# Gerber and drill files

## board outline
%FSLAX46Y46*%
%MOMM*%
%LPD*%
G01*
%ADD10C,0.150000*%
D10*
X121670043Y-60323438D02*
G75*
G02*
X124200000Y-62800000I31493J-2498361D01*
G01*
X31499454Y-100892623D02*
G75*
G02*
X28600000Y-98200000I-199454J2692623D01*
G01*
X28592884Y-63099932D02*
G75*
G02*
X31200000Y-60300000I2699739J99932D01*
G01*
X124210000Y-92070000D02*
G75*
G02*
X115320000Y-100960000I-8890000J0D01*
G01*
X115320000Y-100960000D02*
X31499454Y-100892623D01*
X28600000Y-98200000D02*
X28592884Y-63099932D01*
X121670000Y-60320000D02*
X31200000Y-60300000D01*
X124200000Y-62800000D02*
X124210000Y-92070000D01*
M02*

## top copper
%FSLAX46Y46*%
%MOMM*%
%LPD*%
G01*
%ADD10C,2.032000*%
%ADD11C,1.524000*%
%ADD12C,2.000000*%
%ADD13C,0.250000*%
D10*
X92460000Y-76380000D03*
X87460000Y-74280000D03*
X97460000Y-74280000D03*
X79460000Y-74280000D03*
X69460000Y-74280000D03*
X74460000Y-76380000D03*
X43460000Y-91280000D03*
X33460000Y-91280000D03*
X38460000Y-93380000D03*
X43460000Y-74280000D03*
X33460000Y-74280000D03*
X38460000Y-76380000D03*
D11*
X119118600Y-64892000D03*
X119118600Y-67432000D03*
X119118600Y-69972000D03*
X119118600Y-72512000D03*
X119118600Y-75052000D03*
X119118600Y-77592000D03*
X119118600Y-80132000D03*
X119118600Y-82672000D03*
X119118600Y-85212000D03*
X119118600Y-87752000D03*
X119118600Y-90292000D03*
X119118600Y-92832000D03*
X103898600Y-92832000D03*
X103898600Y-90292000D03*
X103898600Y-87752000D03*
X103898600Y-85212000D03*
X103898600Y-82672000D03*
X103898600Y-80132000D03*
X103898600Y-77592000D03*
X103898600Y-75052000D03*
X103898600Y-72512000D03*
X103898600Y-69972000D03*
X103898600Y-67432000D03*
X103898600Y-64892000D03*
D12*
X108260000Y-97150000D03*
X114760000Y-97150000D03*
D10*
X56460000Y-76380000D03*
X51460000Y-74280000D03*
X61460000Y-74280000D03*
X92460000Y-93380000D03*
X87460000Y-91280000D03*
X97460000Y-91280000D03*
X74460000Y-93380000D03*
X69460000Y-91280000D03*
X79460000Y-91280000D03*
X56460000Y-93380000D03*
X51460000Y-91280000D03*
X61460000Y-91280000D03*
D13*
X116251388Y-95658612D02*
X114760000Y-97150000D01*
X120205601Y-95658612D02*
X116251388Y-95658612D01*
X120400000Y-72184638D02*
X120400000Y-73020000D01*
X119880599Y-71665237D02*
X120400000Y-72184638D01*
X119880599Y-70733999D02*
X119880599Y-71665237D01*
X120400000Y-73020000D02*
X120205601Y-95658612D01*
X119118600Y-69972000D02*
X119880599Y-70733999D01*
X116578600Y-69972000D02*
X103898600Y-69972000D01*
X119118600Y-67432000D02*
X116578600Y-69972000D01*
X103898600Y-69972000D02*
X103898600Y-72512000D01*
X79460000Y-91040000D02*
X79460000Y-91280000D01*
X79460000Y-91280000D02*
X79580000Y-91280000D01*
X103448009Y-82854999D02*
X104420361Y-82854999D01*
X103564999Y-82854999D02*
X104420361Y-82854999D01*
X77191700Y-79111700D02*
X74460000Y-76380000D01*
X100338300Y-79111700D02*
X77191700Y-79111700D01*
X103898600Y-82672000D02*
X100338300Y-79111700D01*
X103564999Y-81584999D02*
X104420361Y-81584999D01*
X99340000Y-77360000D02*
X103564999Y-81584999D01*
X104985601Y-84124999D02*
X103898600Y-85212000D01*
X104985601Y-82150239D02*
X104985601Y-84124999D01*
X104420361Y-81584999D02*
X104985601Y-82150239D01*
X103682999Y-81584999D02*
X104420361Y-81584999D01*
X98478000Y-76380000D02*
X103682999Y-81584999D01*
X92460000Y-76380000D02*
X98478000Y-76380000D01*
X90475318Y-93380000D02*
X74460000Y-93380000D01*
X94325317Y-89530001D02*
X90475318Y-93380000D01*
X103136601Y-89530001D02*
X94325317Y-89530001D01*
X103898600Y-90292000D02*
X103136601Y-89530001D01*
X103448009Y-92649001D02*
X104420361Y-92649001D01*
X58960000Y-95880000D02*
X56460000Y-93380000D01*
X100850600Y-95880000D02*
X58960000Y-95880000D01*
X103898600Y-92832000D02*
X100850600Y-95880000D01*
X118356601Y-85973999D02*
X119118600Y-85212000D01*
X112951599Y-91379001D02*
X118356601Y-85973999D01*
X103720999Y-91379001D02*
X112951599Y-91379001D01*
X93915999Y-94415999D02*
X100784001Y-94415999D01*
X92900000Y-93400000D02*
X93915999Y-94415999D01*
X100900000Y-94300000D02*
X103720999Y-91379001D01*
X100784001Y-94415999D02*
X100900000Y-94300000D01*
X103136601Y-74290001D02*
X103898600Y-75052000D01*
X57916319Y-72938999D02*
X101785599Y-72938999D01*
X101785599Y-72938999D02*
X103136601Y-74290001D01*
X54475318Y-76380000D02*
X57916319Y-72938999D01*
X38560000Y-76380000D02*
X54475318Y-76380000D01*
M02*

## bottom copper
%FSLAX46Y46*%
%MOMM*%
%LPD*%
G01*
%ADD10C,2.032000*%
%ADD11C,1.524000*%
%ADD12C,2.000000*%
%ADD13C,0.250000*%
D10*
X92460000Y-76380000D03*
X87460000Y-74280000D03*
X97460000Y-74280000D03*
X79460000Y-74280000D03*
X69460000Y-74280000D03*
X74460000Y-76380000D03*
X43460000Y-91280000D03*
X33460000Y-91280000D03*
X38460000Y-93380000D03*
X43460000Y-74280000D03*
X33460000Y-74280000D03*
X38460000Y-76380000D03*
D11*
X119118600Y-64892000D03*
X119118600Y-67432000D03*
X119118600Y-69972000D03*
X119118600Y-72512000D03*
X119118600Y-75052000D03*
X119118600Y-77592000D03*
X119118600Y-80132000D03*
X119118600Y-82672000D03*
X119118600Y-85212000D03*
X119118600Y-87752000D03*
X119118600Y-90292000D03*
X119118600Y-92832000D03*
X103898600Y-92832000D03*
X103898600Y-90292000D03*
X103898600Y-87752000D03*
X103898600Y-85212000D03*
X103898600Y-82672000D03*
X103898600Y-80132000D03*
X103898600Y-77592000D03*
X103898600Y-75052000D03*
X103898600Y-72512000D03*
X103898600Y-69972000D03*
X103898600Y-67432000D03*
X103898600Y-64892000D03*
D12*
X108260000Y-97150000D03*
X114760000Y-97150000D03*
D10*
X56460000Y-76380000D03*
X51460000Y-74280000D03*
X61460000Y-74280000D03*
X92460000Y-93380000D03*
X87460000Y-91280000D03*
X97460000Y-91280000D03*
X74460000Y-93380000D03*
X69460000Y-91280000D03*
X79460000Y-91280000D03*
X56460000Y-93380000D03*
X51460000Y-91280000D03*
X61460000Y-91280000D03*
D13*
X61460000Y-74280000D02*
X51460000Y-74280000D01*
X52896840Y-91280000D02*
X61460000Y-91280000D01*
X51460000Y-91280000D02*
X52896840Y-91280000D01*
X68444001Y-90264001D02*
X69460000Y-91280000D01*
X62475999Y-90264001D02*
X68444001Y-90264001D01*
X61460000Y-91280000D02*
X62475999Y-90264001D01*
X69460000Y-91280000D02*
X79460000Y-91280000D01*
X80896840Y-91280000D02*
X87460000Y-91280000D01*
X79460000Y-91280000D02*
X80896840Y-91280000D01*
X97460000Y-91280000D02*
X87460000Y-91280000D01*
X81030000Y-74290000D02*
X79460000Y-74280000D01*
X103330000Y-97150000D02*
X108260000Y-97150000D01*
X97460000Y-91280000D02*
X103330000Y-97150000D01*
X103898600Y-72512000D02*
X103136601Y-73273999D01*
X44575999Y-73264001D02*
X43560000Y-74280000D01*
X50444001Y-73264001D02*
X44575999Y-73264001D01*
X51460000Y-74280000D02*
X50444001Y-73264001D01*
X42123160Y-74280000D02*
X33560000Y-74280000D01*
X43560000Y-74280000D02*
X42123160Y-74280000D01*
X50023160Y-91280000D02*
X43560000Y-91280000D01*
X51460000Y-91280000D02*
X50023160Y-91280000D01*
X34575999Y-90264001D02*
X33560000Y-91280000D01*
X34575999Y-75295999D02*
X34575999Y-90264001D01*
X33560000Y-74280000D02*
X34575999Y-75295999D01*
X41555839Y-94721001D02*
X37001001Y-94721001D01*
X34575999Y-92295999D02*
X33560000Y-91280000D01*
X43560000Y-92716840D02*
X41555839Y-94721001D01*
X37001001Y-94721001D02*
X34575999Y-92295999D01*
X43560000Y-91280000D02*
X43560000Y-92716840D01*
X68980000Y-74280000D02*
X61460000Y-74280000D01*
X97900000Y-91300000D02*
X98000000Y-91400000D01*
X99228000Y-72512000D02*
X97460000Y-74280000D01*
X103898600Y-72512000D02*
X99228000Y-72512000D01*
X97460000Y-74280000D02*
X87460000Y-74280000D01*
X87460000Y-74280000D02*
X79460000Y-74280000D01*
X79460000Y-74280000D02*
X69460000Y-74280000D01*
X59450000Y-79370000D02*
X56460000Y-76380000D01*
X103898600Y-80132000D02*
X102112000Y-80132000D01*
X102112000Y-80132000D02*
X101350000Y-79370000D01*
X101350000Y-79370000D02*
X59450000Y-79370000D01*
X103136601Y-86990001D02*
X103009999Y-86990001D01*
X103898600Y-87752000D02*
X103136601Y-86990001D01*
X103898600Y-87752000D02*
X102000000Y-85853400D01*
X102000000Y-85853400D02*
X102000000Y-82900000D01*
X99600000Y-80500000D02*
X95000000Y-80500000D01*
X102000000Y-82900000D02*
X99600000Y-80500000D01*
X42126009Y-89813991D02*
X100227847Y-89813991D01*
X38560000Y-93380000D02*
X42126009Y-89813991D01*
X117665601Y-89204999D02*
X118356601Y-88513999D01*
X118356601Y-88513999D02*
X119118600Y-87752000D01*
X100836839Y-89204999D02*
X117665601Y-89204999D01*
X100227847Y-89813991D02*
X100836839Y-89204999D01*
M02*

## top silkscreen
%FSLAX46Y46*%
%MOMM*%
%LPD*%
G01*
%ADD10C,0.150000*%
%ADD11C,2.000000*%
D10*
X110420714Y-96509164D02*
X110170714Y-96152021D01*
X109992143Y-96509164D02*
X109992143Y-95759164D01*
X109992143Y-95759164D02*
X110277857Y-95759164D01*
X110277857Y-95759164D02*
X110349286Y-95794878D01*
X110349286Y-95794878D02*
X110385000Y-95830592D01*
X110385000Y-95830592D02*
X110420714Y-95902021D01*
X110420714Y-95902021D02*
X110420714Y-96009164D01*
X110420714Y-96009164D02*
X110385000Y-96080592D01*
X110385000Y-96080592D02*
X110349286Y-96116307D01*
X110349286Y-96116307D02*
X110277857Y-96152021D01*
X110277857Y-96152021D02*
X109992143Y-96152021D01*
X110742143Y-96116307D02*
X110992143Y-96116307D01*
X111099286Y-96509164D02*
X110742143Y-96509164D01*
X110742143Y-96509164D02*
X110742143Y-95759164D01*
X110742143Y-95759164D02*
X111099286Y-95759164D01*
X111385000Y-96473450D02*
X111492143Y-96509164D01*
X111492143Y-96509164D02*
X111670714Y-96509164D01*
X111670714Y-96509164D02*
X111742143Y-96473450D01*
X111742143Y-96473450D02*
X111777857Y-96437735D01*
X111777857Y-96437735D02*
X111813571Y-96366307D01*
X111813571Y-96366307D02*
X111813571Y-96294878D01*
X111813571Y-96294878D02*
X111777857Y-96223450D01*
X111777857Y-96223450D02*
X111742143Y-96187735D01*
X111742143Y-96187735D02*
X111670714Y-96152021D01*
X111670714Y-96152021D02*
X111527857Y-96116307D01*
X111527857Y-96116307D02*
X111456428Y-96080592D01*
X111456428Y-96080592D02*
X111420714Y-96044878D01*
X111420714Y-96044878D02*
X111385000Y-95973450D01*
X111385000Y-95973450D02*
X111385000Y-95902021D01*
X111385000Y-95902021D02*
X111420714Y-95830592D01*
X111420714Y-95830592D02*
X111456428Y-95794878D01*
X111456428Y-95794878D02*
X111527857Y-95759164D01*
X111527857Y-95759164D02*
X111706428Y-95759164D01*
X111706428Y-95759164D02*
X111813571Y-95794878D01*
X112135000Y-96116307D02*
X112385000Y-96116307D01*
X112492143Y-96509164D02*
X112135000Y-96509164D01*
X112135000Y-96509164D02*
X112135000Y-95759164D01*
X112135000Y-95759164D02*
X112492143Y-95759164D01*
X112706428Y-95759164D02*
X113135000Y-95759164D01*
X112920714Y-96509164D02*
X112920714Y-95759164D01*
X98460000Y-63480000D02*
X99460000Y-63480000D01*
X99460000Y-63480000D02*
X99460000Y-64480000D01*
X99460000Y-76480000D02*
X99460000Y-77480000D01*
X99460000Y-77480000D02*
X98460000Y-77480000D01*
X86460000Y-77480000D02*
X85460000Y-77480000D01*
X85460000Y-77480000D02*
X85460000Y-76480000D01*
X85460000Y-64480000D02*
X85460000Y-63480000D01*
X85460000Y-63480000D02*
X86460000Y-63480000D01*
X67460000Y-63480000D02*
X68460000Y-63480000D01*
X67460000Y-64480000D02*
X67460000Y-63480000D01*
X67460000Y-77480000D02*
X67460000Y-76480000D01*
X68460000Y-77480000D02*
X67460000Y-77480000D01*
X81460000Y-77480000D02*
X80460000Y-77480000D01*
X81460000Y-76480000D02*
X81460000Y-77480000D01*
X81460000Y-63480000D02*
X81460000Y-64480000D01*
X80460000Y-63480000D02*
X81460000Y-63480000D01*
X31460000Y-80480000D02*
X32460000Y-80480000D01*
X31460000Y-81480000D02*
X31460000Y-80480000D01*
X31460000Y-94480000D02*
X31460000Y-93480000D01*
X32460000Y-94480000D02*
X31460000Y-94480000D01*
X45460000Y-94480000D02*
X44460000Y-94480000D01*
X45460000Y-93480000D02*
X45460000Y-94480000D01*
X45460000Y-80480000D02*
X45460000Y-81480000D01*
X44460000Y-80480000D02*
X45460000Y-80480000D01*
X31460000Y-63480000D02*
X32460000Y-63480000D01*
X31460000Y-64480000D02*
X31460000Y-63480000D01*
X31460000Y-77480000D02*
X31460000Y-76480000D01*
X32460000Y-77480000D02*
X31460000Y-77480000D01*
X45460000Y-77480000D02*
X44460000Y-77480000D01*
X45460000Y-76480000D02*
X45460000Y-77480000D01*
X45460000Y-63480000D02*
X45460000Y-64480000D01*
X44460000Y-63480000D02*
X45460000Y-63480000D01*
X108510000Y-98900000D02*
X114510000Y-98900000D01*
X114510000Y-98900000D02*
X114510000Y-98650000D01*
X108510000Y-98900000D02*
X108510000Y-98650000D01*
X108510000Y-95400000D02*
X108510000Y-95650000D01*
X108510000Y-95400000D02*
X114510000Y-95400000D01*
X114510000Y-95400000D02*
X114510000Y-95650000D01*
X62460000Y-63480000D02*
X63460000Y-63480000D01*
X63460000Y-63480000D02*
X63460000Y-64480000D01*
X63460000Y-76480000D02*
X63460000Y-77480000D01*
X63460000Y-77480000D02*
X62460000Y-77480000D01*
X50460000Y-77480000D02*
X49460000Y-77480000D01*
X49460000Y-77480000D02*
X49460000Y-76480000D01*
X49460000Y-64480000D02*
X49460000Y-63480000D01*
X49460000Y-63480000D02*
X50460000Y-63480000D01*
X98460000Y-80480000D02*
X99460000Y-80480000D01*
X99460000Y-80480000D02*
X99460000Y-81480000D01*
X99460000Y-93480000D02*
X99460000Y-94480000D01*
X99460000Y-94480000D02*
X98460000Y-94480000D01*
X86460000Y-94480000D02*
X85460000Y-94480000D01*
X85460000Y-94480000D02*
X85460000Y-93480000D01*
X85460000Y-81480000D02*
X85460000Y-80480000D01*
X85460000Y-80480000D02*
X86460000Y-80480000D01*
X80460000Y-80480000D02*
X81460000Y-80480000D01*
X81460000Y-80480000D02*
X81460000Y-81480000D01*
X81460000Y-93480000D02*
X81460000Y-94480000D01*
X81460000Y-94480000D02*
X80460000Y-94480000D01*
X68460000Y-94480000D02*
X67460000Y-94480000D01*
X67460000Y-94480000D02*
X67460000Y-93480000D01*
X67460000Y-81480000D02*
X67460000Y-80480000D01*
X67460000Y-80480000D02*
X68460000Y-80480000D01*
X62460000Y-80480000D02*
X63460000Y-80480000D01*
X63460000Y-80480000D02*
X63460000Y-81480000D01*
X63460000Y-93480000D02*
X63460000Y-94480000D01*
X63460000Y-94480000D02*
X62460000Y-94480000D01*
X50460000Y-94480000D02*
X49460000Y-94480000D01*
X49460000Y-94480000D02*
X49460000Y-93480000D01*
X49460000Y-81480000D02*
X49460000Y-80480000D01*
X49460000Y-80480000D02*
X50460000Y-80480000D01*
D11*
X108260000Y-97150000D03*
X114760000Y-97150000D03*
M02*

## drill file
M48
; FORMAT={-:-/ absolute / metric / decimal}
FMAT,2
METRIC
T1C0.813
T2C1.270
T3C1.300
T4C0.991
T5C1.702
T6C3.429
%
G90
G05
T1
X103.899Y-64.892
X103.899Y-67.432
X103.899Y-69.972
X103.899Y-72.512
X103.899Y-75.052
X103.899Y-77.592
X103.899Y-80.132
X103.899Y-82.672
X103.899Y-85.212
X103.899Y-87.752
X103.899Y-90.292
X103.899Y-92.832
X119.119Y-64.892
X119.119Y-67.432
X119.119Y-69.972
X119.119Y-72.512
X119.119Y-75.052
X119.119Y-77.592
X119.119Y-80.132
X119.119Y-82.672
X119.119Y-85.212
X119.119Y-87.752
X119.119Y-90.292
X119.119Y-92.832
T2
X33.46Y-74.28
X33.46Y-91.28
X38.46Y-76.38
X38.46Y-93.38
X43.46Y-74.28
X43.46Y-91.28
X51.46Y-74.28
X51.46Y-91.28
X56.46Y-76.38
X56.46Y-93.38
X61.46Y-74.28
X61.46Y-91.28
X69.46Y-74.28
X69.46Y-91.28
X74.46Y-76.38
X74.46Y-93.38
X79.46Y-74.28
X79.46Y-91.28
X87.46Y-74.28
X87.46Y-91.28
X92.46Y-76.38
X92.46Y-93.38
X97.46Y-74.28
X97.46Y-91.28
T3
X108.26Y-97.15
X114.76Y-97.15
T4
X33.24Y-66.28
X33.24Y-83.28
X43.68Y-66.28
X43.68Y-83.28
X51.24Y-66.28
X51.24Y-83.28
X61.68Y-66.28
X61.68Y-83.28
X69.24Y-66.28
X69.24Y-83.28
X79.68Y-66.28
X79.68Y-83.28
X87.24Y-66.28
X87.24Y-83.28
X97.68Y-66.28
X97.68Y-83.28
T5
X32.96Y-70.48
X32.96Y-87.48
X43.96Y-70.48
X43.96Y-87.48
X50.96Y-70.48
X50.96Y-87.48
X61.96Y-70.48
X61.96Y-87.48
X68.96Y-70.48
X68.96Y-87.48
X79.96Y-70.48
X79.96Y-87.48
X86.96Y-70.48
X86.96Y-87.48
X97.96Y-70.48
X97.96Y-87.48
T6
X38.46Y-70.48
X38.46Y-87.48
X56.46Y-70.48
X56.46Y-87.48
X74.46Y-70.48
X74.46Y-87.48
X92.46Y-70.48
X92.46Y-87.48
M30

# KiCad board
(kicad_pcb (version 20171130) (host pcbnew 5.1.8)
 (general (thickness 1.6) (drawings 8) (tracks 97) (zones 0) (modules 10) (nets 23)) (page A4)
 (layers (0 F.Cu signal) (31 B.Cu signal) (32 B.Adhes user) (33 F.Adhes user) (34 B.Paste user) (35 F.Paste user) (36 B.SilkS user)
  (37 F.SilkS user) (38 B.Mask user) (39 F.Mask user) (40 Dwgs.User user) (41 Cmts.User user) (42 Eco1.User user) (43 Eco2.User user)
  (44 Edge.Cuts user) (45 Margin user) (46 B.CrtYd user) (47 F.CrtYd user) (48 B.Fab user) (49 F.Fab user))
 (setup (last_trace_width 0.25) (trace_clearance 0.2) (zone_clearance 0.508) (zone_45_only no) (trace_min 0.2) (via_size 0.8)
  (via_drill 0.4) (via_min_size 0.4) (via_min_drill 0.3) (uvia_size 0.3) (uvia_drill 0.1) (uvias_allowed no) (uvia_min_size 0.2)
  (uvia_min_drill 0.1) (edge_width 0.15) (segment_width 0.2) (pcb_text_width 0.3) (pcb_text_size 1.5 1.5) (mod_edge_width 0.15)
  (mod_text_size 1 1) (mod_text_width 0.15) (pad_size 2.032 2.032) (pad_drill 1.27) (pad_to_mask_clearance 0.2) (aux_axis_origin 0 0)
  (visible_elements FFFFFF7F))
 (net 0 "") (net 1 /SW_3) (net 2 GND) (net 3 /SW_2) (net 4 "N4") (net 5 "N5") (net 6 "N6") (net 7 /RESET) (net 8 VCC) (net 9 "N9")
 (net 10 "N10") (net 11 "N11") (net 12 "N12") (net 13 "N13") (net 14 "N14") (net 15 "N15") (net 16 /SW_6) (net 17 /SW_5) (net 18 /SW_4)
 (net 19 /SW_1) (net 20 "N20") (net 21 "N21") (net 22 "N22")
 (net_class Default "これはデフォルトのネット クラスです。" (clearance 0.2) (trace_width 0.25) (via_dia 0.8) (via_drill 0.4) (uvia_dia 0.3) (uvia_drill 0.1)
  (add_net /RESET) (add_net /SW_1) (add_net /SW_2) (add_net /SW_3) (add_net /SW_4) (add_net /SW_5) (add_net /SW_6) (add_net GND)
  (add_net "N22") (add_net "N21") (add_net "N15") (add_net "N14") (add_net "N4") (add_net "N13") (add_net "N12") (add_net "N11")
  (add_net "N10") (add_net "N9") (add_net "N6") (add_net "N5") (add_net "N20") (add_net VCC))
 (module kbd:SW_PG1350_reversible (layer F.Cu) (at 92.46 70.48)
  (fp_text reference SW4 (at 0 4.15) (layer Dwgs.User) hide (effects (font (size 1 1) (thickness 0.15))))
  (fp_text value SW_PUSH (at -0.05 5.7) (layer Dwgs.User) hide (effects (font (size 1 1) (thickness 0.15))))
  (fp_line (start 6 -7) (end 7 -7) (layer F.SilkS) (width 0.15))
  (fp_line (start 7 -7) (end 7 -6) (layer F.SilkS) (width 0.15)) (fp_line (start 7 6) (end 7 7) (layer F.SilkS) (width 0.15))
  (fp_line (start 7 7) (end 6 7) (layer F.SilkS) (width 0.15))
  (fp_line (start -6 7) (end -7 7) (layer F.SilkS) (width 0.15))
  (fp_line (start -7 7) (end -7 6) (layer F.SilkS) (width 0.15))
  (fp_line (start -7 -6) (end -7 -7) (layer F.SilkS) (width 0.15))
  (fp_line (start -7 -7) (end -6 -7) (layer F.SilkS) (width 0.15))
  (pad "" np_thru_hole circle (at -5.5 0) (size 1.7018 1.7018) (drill 1.7018) (layers *.Cu *.Mask))
  (pad "" np_thru_hole circle (at 5.5 0) (size 1.7018 1.7018) (drill 1.7018) (layers *.Cu *.Mask))
  (pad "" np_thru_hole circle (at 5.22 -4.2) (size 0.9906 0.9906) (drill 0.9906) (layers *.Cu *.Mask))
  (pad 1 thru_hole circle (at 0 5.9) (size 2.032 2.032) (drill 1.27) (layers *.Cu *.Mask) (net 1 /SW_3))
  (pad 2 thru_hole circle (at -5 3.8) (size 2.032 2.032) (drill 1.27) (layers *.Cu *.Mask) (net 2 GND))
  (pad "" np_thru_hole circle (at 0 0) (size 3.429 3.429) (drill 3.429) (layers *.Cu *.Mask))
  (pad 2 thru_hole circle (at 5 3.8) (size 2.032 2.032) (drill 1.27) (layers *.Cu *.Mask) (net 2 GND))
  (pad "" np_thru_hole circle (at -5.22 -4.2) (size 0.9906 0.9906) (drill 0.9906) (layers *.Cu *.Mask)))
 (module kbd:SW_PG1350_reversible (layer F.Cu) (at 74.46 70.48)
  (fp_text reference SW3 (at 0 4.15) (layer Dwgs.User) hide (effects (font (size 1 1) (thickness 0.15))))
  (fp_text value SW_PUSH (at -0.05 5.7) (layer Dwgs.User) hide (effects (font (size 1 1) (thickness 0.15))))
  (fp_line (start -7 -7) (end -6 -7) (layer F.SilkS) (width 0.15))
  (fp_line (start -7 -6) (end -7 -7) (layer F.SilkS) (width 0.15))
  (fp_line (start -7 7) (end -7 6) (layer F.SilkS) (width 0.15))
  (fp_line (start -6 7) (end -7 7) (layer F.SilkS) (width 0.15)) (fp_line (start 7 7) (end 6 7) (layer F.SilkS) (width 0.15))
  (fp_line (start 7 6) (end 7 7) (layer F.SilkS) (width 0.15))
  (fp_line (start 7 -7) (end 7 -6) (layer F.SilkS) (width 0.15))
  (fp_line (start 6 -7) (end 7 -7) (layer F.SilkS) (width 0.15))
  (pad "" np_thru_hole circle (at -5.22 -4.2) (size 0.9906 0.9906) (drill 0.9906) (layers *.Cu *.Mask))
  (pad 2 thru_hole circle (at 5 3.8) (size 2.032 2.032) (drill 1.27) (layers *.Cu *.Mask) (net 2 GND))
  (pad "" np_thru_hole circle (at 0 0) (size 3.429 3.429) (drill 3.429) (layers *.Cu *.Mask))
  (pad 2 thru_hole circle (at -5 3.8) (size 2.032 2.032) (drill 1.27) (layers *.Cu *.Mask) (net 2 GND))
  (pad 1 thru_hole circle (at 0 5.9) (size 2.032 2.032) (drill 1.27) (layers *.Cu *.Mask) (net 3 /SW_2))
  (pad "" np_thru_hole circle (at 5.22 -4.2) (size 0.9906 0.9906) (drill 0.9906) (layers *.Cu *.Mask))
  (pad "" np_thru_hole circle (at 5.5 0) (size 1.7018 1.7018) (drill 1.7018) (layers *.Cu *.Mask))
  (pad "" np_thru_hole circle (at -5.5 0) (size 1.7018 1.7018) (drill 1.7018) (layers *.Cu *.Mask)))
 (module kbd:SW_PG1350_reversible (layer F.Cu) (at 38.46 87.48)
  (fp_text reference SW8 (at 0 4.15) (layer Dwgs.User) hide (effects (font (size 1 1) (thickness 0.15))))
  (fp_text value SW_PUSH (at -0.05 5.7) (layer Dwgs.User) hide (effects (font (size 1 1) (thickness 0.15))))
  (fp_line (start -7 -7) (end -6 -7) (layer F.SilkS) (width 0.15))
  (fp_line (start -7 -6) (end -7 -7) (layer F.SilkS) (width 0.15))
  (fp_line (start -7 7) (end -7 6) (layer F.SilkS) (width 0.15))
  (fp_line (start -6 7) (end -7 7) (layer F.SilkS) (width 0.15)) (fp_line (start 7 7) (end 6 7) (layer F.SilkS) (width 0.15))
  (fp_line (start 7 6) (end 7 7) (layer F.SilkS) (width 0.15))
  (fp_line (start 7 -7) (end 7 -6) (layer F.SilkS) (width 0.15))
  (fp_line (start 6 -7) (end 7 -7) (layer F.SilkS) (width 0.15))
  (pad "" np_thru_hole circle (at -5.22 -4.2) (size 0.9906 0.9906) (drill 0.9906) (layers *.Cu *.Mask))
  (pad 2 thru_hole circle (at 5 3.8) (size 2.032 2.032) (drill 1.27) (layers *.Cu *.Mask) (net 2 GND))
  (pad "" np_thru_hole circle (at 0 0) (size 3.429 3.429) (drill 3.429) (layers *.Cu *.Mask))
  (pad 2 thru_hole circle (at -5 3.8) (size 2.032 2.032) (drill 1.27) (layers *.Cu *.Mask) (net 2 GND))
  (pad 1 thru_hole circle (at 0 5.9) (size 2.032 2.032) (drill 1.27) (layers *.Cu *.Mask) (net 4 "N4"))
  (pad "" np_thru_hole circle (at 5.22 -4.2) (size 0.9906 0.9906) (drill 0.9906) (layers *.Cu *.Mask))
  (pad "" np_thru_hole circle (at 5.5 0) (size 1.7018 1.7018) (drill 1.7018) (layers *.Cu *.Mask))
  (pad "" np_thru_hole circle (at -5.5 0) (size 1.7018 1.7018) (drill 1.7018) (layers *.Cu *.Mask)))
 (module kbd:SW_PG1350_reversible (layer F.Cu) (at 38.46 70.48)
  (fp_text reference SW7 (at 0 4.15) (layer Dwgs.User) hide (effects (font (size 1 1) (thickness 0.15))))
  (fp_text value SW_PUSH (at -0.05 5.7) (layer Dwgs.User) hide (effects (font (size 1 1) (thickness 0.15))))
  (fp_line (start -7 -7) (end -6 -7) (layer F.SilkS) (width 0.15))
  (fp_line (start -7 -6) (end -7 -7) (layer F.SilkS) (width 0.15))
  (fp_line (start -7 7) (end -7 6) (layer F.SilkS) (width 0.15))
  (fp_line (start -6 7) (end -7 7) (layer F.SilkS) (width 0.15)) (fp_line (start 7 7) (end 6 7) (layer F.SilkS) (width 0.15))
  (fp_line (start 7 6) (end 7 7) (layer F.SilkS) (width 0.15))
  (fp_line (start 7 -7) (end 7 -6) (layer F.SilkS) (width 0.15))
  (fp_line (start 6 -7) (end 7 -7) (layer F.SilkS) (width 0.15))
  (pad "" np_thru_hole circle (at -5.22 -4.2) (size 0.9906 0.9906) (drill 0.9906) (layers *.Cu *.Mask))
  (pad 2 thru_hole circle (at 5 3.8) (size 2.032 2.032) (drill 1.27) (layers *.Cu *.Mask) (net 2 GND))
  (pad "" np_thru_hole circle (at 0 0) (size 3.429 3.429) (drill 3.429) (layers *.Cu *.Mask))
  (pad 2 thru_hole circle (at -5 3.8) (size 2.032 2.032) (drill 1.27) (layers *.Cu *.Mask) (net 2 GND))
  (pad 1 thru_hole circle (at 0 5.9) (size 2.032 2.032) (drill 1.27) (layers *.Cu *.Mask) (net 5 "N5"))
  (pad "" np_thru_hole circle (at 5.22 -4.2) (size 0.9906 0.9906) (drill 0.9906) (layers *.Cu *.Mask))
  (pad "" np_thru_hole circle (at 5.5 0) (size 1.7018 1.7018) (drill 1.7018) (layers *.Cu *.Mask))
  (pad "" np_thru_hole circle (at -5.5 0) (size 1.7018 1.7018) (drill 1.7018) (layers *.Cu *.Mask)))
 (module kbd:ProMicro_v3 (layer B.Cu) (at 111.51 79.37 180)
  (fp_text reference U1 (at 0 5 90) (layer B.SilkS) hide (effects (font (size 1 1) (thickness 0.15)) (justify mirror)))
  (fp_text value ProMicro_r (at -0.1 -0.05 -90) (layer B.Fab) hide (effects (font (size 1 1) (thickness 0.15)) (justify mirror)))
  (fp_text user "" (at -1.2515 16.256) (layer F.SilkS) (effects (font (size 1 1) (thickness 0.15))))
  (pad 24 thru_hole circle (at -7.6086 14.478 180) (size 1.524 1.524) (drill 0.8128) (layers *.Cu *.Mask B.SilkS) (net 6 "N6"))
  (pad 23 thru_hole circle (at -7.6086 11.938 180) (size 1.524 1.524) (drill 0.8128) (layers *.Cu *.Mask B.SilkS) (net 2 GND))
  (pad 22 thru_hole circle (at -7.6086 9.398 180) (size 1.524 1.524) (drill 0.8128) (layers *.Cu *.Mask B.SilkS) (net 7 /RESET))
  (pad 21 thru_hole circle (at -7.6086 6.858 180) (size 1.524 1.524) (drill 0.8128) (layers *.Cu *.Mask B.SilkS) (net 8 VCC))
  (pad 20 thru_hole circle (at -7.6086 4.318 180) (size 1.524 1.524) (drill 0.8128) (layers *.Cu *.Mask B.SilkS) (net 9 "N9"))
  (pad 19 thru_hole circle (at -7.6086 1.778 180) (size 1.524 1.524) (drill 0.8128) (layers *.Cu *.Mask B.SilkS) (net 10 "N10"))
  (pad 18 thru_hole circle (at -7.6086 -0.762 180) (size 1.524 1.524) (drill 0.8128) (layers *.Cu *.Mask B.SilkS) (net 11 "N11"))
  (pad 17 thru_hole circle (at -7.6086 -3.302 180) (size 1.524 1.524) (drill 0.8128) (layers *.Cu *.Mask B.SilkS) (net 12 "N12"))
  (pad 16 thru_hole circle (at -7.6086 -5.842 180) (size 1.524 1.524) (drill 0.8128) (layers *.Cu *.Mask B.SilkS) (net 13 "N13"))
  (pad 15 thru_hole circle (at -7.6086 -8.382 180) (size 1.524 1.524) (drill 0.8128) (layers *.Cu *.Mask B.SilkS) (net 4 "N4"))
  (pad 14 thru_hole circle (at -7.6086 -10.922 180) (size 1.524 1.524) (drill 0.8128) (layers *.Cu *.Mask B.SilkS) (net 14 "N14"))
  (pad 13 thru_hole circle (at -7.6086 -13.462 180) (size 1.524 1.524) (drill 0.8128) (layers *.Cu *.Mask B.SilkS) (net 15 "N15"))
  (pad 12 thru_hole circle (at 7.6114 -13.462 180) (size 1.524 1.524) (drill 0.8128) (layers *.Cu *.Mask B.SilkS) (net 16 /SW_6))
  (pad 11 thru_hole circle (at 7.6114 -10.922 180) (size 1.524 1.524) (drill 0.8128) (layers *.Cu *.Mask B.SilkS) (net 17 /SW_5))
  (pad 10 thru_hole circle (at 7.6114 -8.382 180) (size 1.524 1.524) (drill 0.8128) (layers *.Cu *.Mask B.SilkS) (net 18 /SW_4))
  (pad 9 thru_hole circle (at 7.6114 -5.842 180) (size 1.524 1.524) (drill 0.8128) (layers *.Cu *.Mask B.SilkS) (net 1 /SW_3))
  (pad 8 thru_hole circle (at 7.6114 -3.302 180) (size 1.524 1.524) (drill 0.8128) (layers *.Cu *.Mask B.SilkS) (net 3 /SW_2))
  (pad 7 thru_hole circle (at 7.6114 -0.762 180) (size 1.524 1.524) (drill 0.8128) (layers *.Cu *.Mask B.SilkS) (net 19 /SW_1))
  (pad 6 thru_hole circle (at 7.6114 1.778 180) (size 1.524 1.524) (drill 0.8128) (layers *.Cu *.Mask B.SilkS) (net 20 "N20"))
  (pad 5 thru_hole circle (at 7.6114 4.318 180) (size 1.524 1.524) (drill 0.8128) (layers *.Cu *.Mask B.SilkS) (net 5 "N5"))
  (pad 4 thru_hole circle (at 7.6114 6.858 180) (size 1.524 1.524) (drill 0.8128) (layers *.Cu *.Mask B.SilkS) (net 2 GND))
  (pad 3 thru_hole circle (at 7.6114 9.398 180) (size 1.524 1.524) (drill 0.8128) (layers *.Cu *.Mask B.SilkS) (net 2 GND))
  (pad 2 thru_hole circle (at 7.6114 11.938 180) (size 1.524 1.524) (drill 0.8128) (layers *.Cu *.Mask B.SilkS) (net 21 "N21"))
  (pad 1 thru_hole circle (at 7.6114 14.478 180) (size 1.524 1.524) (drill 0.8128) (layers *.Cu *.Mask B.SilkS) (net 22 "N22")))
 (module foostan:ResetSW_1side (layer F.Cu) (at 111.51 97.15)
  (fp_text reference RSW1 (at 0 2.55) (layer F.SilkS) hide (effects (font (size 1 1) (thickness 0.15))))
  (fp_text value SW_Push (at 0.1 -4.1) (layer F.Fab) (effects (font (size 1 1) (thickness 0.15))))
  (fp_line (start -3 1.75) (end 3 1.75) (layer F.SilkS) (width 0.15))
  (fp_line (start 3 1.75) (end 3 1.5) (layer F.SilkS) (width 0.15))
  (fp_line (start -3 1.75) (end -3 1.5) (layer F.SilkS) (width 0.15))
  (fp_line (start -3 -1.75) (end -3 -1.5) (layer F.SilkS) (width 0.15))
  (fp_line (start -3 -1.75) (end 3 -1.75) (layer F.SilkS) (width 0.15))
  (fp_line (start 3 -1.75) (end 3 -1.5) (layer F.SilkS) (width 0.15))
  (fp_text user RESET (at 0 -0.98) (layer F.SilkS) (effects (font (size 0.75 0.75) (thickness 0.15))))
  (pad 2 thru_hole circle (at -3.25 0) (size 2 2) (drill 1.3) (layers *.Cu F.SilkS B.Mask) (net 2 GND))
  (pad 1 thru_hole circle (at 3.25 0) (size 2 2) (drill 1.3) (layers *.Cu F.SilkS B.Mask) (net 7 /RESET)))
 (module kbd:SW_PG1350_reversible (layer F.Cu) (at 56.46 70.48)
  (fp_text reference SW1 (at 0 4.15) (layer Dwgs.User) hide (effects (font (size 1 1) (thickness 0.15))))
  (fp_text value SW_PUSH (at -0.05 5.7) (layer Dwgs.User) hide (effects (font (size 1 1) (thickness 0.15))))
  (fp_line (start 6 -7) (end 7 -7) (layer F.SilkS) (width 0.15))
  (fp_line (start 7 -7) (end 7 -6) (layer F.SilkS) (width 0.15)) (fp_line (start 7 6) (end 7 7) (layer F.SilkS) (width 0.15))
  (fp_line (start 7 7) (end 6 7) (layer F.SilkS) (width 0.15))
  (fp_line (start -6 7) (end -7 7) (layer F.SilkS) (width 0.15))
  (fp_line (start -7 7) (end -7 6) (layer F.SilkS) (width 0.15))
  (fp_line (start -7 -6) (end -7 -7) (layer F.SilkS) (width 0.15))
  (fp_line (start -7 -7) (end -6 -7) (layer F.SilkS) (width 0.15))
  (pad "" np_thru_hole circle (at -5.5 0) (size 1.7018 1.7018) (drill 1.7018) (layers *.Cu *.Mask))
  (pad "" np_thru_hole circle (at 5.5 0) (size 1.7018 1.7018) (drill 1.7018) (layers *.Cu *.Mask))
  (pad "" np_thru_hole circle (at 5.22 -4.2) (size 0.9906 0.9906) (drill 0.9906) (layers *.Cu *.Mask))
  (pad 1 thru_hole circle (at 0 5.9) (size 2.032 2.032) (drill 1.27) (layers *.Cu *.Mask) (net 19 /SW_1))
  (pad 2 thru_hole circle (at -5 3.8) (size 2.032 2.032) (drill 1.27) (layers *.Cu *.Mask) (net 2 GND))
  (pad "" np_thru_hole circle (at 0 0) (size 3.429 3.429) (drill 3.429) (layers *.Cu *.Mask))
  (pad 2 thru_hole circle (at 5 3.8) (size 2.032 2.032) (drill 1.27) (layers *.Cu *.Mask) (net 2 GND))
  (pad "" np_thru_hole circle (at -5.22 -4.2) (size 0.9906 0.9906) (drill 0.9906) (layers *.Cu *.Mask)))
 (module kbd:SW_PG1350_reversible (layer F.Cu) (at 92.46 87.48)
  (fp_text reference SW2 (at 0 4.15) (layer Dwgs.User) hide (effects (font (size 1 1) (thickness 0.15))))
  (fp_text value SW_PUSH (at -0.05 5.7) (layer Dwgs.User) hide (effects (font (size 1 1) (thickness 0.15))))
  (fp_line (start 6 -7) (end 7 -7) (layer F.SilkS) (width 0.15))
  (fp_line (start 7 -7) (end 7 -6) (layer F.SilkS) (width 0.15)) (fp_line (start 7 6) (end 7 7) (layer F.SilkS) (width 0.15))
  (fp_line (start 7 7) (end 6 7) (layer F.SilkS) (width 0.15))
  (fp_line (start -6 7) (end -7 7) (layer F.SilkS) (width 0.15))
  (fp_line (start -7 7) (end -7 6) (layer F.SilkS) (width 0.15))
  (fp_line (start -7 -6) (end -7 -7) (layer F.SilkS) (width 0.15))
  (fp_line (start -7 -7) (end -6 -7) (layer F.SilkS) (width 0.15))
  (pad "" np_thru_hole circle (at -5.5 0) (size 1.7018 1.7018) (drill 1.7018) (layers *.Cu *.Mask))
  (pad "" np_thru_hole circle (at 5.5 0) (size 1.7018 1.7018) (drill 1.7018) (layers *.Cu *.Mask))
  (pad "" np_thru_hole circle (at 5.22 -4.2) (size 0.9906 0.9906) (drill 0.9906) (layers *.Cu *.Mask))
  (pad 1 thru_hole circle (at 0 5.9) (size 2.032 2.032) (drill 1.27) (layers *.Cu *.Mask) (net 13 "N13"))
  (pad 2 thru_hole circle (at -5 3.8) (size 2.032 2.032) (drill 1.27) (layers *.Cu *.Mask) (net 2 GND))
  (pad "" np_thru_hole circle (at 0 0) (size 3.429 3.429) (drill 3.429) (layers *.Cu *.Mask))
  (pad 2 thru_hole circle (at 5 3.8) (size 2.032 2.032) (drill 1.27) (layers *.Cu *.Mask) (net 2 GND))
  (pad "" np_thru_hole circle (at -5.22 -4.2) (size 0.9906 0.9906) (drill 0.9906) (layers *.Cu *.Mask)))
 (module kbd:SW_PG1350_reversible (layer F.Cu) (at 74.46 87.48)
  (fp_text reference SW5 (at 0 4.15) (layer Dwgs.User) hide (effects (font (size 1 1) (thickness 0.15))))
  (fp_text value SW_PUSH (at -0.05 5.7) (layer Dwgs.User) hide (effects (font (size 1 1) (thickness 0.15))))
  (fp_line (start 6 -7) (end 7 -7) (layer F.SilkS) (width 0.15))
  (fp_line (start 7 -7) (end 7 -6) (layer F.SilkS) (width 0.15)) (fp_line (start 7 6) (end 7 7) (layer F.SilkS) (width 0.15))
  (fp_line (start 7 7) (end 6 7) (layer F.SilkS) (width 0.15))
  (fp_line (start -6 7) (end -7 7) (layer F.SilkS) (width 0.15))
  (fp_line (start -7 7) (end -7 6) (layer F.SilkS) (width 0.15))
  (fp_line (start -7 -6) (end -7 -7) (layer F.SilkS) (width 0.15))
  (fp_line (start -7 -7) (end -6 -7) (layer F.SilkS) (width 0.15))
  (pad "" np_thru_hole circle (at -5.5 0) (size 1.7018 1.7018) (drill 1.7018) (layers *.Cu *.Mask))
  (pad "" np_thru_hole circle (at 5.5 0) (size 1.7018 1.7018) (drill 1.7018) (layers *.Cu *.Mask))
  (pad "" np_thru_hole circle (at 5.22 -4.2) (size 0.9906 0.9906) (drill 0.9906) (layers *.Cu *.Mask))
  (pad 1 thru_hole circle (at 0 5.9) (size 2.032 2.032) (drill 1.27) (layers *.Cu *.Mask) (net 17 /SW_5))
  (pad 2 thru_hole circle (at -5 3.8) (size 2.032 2.032) (drill 1.27) (layers *.Cu *.Mask) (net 2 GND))
  (pad "" np_thru_hole circle (at 0 0) (size 3.429 3.429) (drill 3.429) (layers *.Cu *.Mask))
  (pad 2 thru_hole circle (at 5 3.8) (size 2.032 2.032) (drill 1.27) (layers *.Cu *.Mask) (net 2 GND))
  (pad "" np_thru_hole circle (at -5.22 -4.2) (size 0.9906 0.9906) (drill 0.9906) (layers *.Cu *.Mask)))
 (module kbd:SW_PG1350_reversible (layer F.Cu) (at 56.46 87.48)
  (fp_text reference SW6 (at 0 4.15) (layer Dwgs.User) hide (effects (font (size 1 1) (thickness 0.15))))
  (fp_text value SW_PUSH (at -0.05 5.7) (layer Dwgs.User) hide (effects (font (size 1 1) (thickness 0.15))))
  (fp_line (start 6 -7) (end 7 -7) (layer F.SilkS) (width 0.15))
  (fp_line (start 7 -7) (end 7 -6) (layer F.SilkS) (width 0.15)) (fp_line (start 7 6) (end 7 7) (layer F.SilkS) (width 0.15))
  (fp_line (start 7 7) (end 6 7) (layer F.SilkS) (width 0.15))
  (fp_line (start -6 7) (end -7 7) (layer F.SilkS) (width 0.15))
  (fp_line (start -7 7) (end -7 6) (layer F.SilkS) (width 0.15))
  (fp_line (start -7 -6) (end -7 -7) (layer F.SilkS) (width 0.15))
  (fp_line (start -7 -7) (end -6 -7) (layer F.SilkS) (width 0.15))
  (pad "" np_thru_hole circle (at -5.5 0) (size 1.7018 1.7018) (drill 1.7018) (layers *.Cu *.Mask))
  (pad "" np_thru_hole circle (at 5.5 0) (size 1.7018 1.7018) (drill 1.7018) (layers *.Cu *.Mask))
  (pad "" np_thru_hole circle (at 5.22 -4.2) (size 0.9906 0.9906) (drill 0.9906) (layers *.Cu *.Mask))
  (pad 1 thru_hole circle (at 0 5.9) (size 2.032 2.032) (drill 1.27) (layers *.Cu *.Mask) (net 16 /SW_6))
  (pad 2 thru_hole circle (at -5 3.8) (size 2.032 2.032) (drill 1.27) (layers *.Cu *.Mask) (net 2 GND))
  (pad "" np_thru_hole circle (at 0 0) (size 3.429 3.429) (drill 3.429) (layers *.Cu *.Mask))
  (pad 2 thru_hole circle (at 5 3.8) (size 2.032 2.032) (drill 1.27) (layers *.Cu *.Mask) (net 2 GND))
  (pad "" np_thru_hole circle (at -5.22 -4.2) (size 0.9906 0.9906) (drill 0.9906) (layers *.Cu *.Mask)))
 (gr_arc (start 121.701536 62.821799) (end 124.2 62.8) (angle -90.22231091) (layer Edge.Cuts) (width 0.15))
 (gr_arc (start 31.3 98.2) (end 28.6 98.2) (angle -94.2363948) (layer Edge.Cuts) (width 0.15))
 (gr_arc (start 31.292623 63) (end 31.2 60.3) (angle -90.15510012) (layer Edge.Cuts) (width 0.15))
 (gr_arc (start 115.32 92.07) (end 115.32 100.96) (angle -90) (layer Edge.Cuts) (width 0.15))
 (gr_line (start 115.32 100.96) (end 31.499454 100.892623) (layer Edge.Cuts) (width 0.15))
 (gr_line (start 28.6 98.2) (end 28.592884 63.099932) (layer Edge.Cuts) (width 0.15))
 (gr_line (start 121.67 60.32) (end 31.2 60.3) (layer Edge.Cuts) (width 0.15))
 (gr_line (start 124.2 62.8) (end 124.21 92.07) (layer Edge.Cuts) (width 0.15))
 (segment (start 116.251388 95.658612) (end 114.76 97.15) (width 0.25) (layer F.Cu) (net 7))
 (segment (start 120.205601 95.658612) (end 116.251388 95.658612) (width 0.25) (layer F.Cu) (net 7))
 (segment (start 120.4 72.184638) (end 120.4 73.02) (width 0.25) (layer F.Cu) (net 7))
 (segment (start 119.880599 71.665237) (end 120.4 72.184638) (width 0.25) (layer F.Cu) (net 7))
 (segment (start 119.880599 70.733999) (end 119.880599 71.665237) (width 0.25) (layer F.Cu) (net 7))
 (segment (start 120.4 73.02) (end 120.205601 95.658612) (width 0.25) (layer F.Cu) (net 7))
 (segment (start 119.1186 69.972) (end 119.880599 70.733999) (width 0.25) (layer F.Cu) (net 7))
 (segment (start 61.46 74.28) (end 51.46 74.28) (width 0.25) (layer B.Cu) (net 2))
 (segment (start 52.89684 91.28) (end 61.46 91.28) (width 0.25) (layer B.Cu) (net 2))
 (segment (start 51.46 91.28) (end 52.89684 91.28) (width 0.25) (layer B.Cu) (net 2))
 (segment (start 68.444001 90.264001) (end 69.46 91.28) (width 0.25) (layer B.Cu) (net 2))
 (segment (start 62.475999 90.264001) (end 68.444001 90.264001) (width 0.25) (layer B.Cu) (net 2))
 (segment (start 61.46 91.28) (end 62.475999 90.264001) (width 0.25) (layer B.Cu) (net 2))
 (segment (start 69.46 91.28) (end 79.46 91.28) (width 0.25) (layer B.Cu) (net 2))
 (segment (start 80.89684 91.28) (end 87.46 91.28) (width 0.25) (layer B.Cu) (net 2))
 (segment (start 79.46 91.28) (end 80.89684 91.28) (width 0.25) (layer B.Cu) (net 2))
 (segment (start 97.46 91.28) (end 87.46 91.28) (width 0.25) (layer B.Cu) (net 2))
 (segment (start 81.03 74.29) (end 79.46 74.28) (width 0.25) (layer B.Cu) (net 2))
 (segment (start 103.33 97.15) (end 108.26 97.15) (width 0.25) (layer B.Cu) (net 2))
 (segment (start 97.46 91.28) (end 103.33 97.15) (width 0.25) (layer B.Cu) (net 2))
 (segment (start 103.8986 72.512) (end 103.136601 73.273999) (width 0.25) (layer B.Cu) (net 2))
 (segment (start 116.5786 69.972) (end 103.8986 69.972) (width 0.25) (layer F.Cu) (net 2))
 (segment (start 119.1186 67.432) (end 116.5786 69.972) (width 0.25) (layer F.Cu) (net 2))
 (segment (start 103.8986 69.972) (end 103.8986 72.512) (width 0.25) (layer F.Cu) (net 2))
 (segment (start 44.575999 73.264001) (end 43.56 74.28) (width 0.25) (layer B.Cu) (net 2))
 (segment (start 50.444001 73.264001) (end 44.575999 73.264001) (width 0.25) (layer B.Cu) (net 2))
 (segment (start 51.46 74.28) (end 50.444001 73.264001) (width 0.25) (layer B.Cu) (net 2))
 (segment (start 42.12316 74.28) (end 33.56 74.28) (width 0.25) (layer B.Cu) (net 2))
 (segment (start 43.56 74.28) (end 42.12316 74.28) (width 0.25) (layer B.Cu) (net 2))
 (segment (start 50.02316 91.28) (end 43.56 91.28) (width 0.25) (layer B.Cu) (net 2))
 (segment (start 51.46 91.28) (end 50.02316 91.28) (width 0.25) (layer B.Cu) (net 2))
 (segment (start 34.575999 90.264001) (end 33.56 91.28) (width 0.25) (layer B.Cu) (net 2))
 (segment (start 34.575999 75.295999) (end 34.575999 90.264001) (width 0.25) (layer B.Cu) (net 2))
 (segment (start 33.56 74.28) (end 34.575999 75.295999) (width 0.25) (layer B.Cu) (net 2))
 (segment (start 41.555839 94.721001) (end 37.001001 94.721001) (width 0.25) (layer B.Cu) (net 2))
 (segment (start 34.575999 92.295999) (end 33.56 91.28) (width 0.25) (layer B.Cu) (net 2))
 (segment (start 43.56 92.71684) (end 41.555839 94.721001) (width 0.25) (layer B.Cu) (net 2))
 (segment (start 37.001001 94.721001) (end 34.575999 92.295999) (width 0.25) (layer B.Cu) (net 2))
 (segment (start 43.56 91.28) (end 43.56 92.71684) (width 0.25) (layer B.Cu) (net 2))
 (segment (start 79.46 91.04) (end 79.46 91.28) (width 0.25) (layer F.Cu) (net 2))
 (segment (start 79.46 91.28) (end 79.58 91.28) (width 0.25) (layer F.Cu) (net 2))
 (segment (start 68.98 74.28) (end 61.46 74.28) (width 0.25) (layer B.Cu) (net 2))
 (segment (start 97.9 91.3) (end 98 91.4) (width 0.25) (layer B.Cu) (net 2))
 (segment (start 99.228 72.512) (end 97.46 74.28) (width 0.25) (layer B.Cu) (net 2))
 (segment (start 103.8986 72.512) (end 99.228 72.512) (width 0.25) (layer B.Cu) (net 2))
 (segment (start 97.46 74.28) (end 87.46 74.28) (width 0.25) (layer B.Cu) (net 2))
 (segment (start 87.46 74.28) (end 79.46 74.28) (width 0.25) (layer B.Cu) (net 2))
 (segment (start 79.46 74.28) (end 69.46 74.28) (width 0.25) (layer B.Cu) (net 2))
 (segment (start 59.45 79.37) (end 56.46 76.38) (width 0.25) (layer B.Cu) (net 19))
 (segment (start 103.8986 80.132) (end 102.112 80.132) (width 0.25) (layer B.Cu) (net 19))
 (segment (start 102.112 80.132) (end 101.35 79.37) (width 0.25) (layer B.Cu) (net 19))
 (segment (start 101.35 79.37) (end 59.45 79.37) (width 0.25) (layer B.Cu) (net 19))
 (segment (start 103.448009 82.854999) (end 104.420361 82.854999) (width 0.25) (layer F.Cu) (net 3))
 (segment (start 103.564999 82.854999) (end 104.420361 82.854999) (width 0.25) (layer F.Cu) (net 3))
 (segment (start 77.1917 79.1117) (end 74.46 76.38) (width 0.25) (layer F.Cu) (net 3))
 (segment (start 100.3383 79.1117) (end 77.1917 79.1117) (width 0.25) (layer F.Cu) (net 3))
 (segment (start 103.8986 82.672) (end 100.3383 79.1117) (width 0.25) (layer F.Cu) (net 3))
 (segment (start 103.564999 81.584999) (end 104.420361 81.584999) (width 0.25) (layer F.Cu) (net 1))
 (segment (start 99.34 77.36) (end 103.564999 81.584999) (width 0.25) (layer F.Cu) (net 1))
 (segment (start 104.985601 84.124999) (end 103.8986 85.212) (width 0.25) (layer F.Cu) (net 1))
 (segment (start 104.985601 82.150239) (end 104.985601 84.124999) (width 0.25) (layer F.Cu) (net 1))
 (segment (start 104.420361 81.584999) (end 104.985601 82.150239) (width 0.25) (layer F.Cu) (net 1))
 (segment (start 103.682999 81.584999) (end 104.420361 81.584999) (width 0.25) (layer F.Cu) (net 1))
 (segment (start 98.478 76.38) (end 103.682999 81.584999) (width 0.25) (layer F.Cu) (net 1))
 (segment (start 92.46 76.38) (end 98.478 76.38) (width 0.25) (layer F.Cu) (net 1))
 (segment (start 103.136601 86.990001) (end 103.009999 86.990001) (width 0.25) (layer B.Cu) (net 18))
 (segment (start 103.8986 87.752) (end 103.136601 86.990001) (width 0.25) (layer B.Cu) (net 18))
 (segment (start 103.8986 87.752) (end 102 85.8534) (width 0.25) (layer B.Cu) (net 18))
 (segment (start 102 85.8534) (end 102 82.9) (width 0.25) (layer B.Cu) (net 18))
 (segment (start 99.6 80.5) (end 95 80.5) (width 0.25) (layer B.Cu) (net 18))
 (segment (start 102 82.9) (end 99.6 80.5) (width 0.25) (layer B.Cu) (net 18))
 (segment (start 90.475318 93.38) (end 74.46 93.38) (width 0.25) (layer F.Cu) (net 17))
 (segment (start 94.325317 89.530001) (end 90.475318 93.38) (width 0.25) (layer F.Cu) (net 17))
 (segment (start 103.136601 89.530001) (end 94.325317 89.530001) (width 0.25) (layer F.Cu) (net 17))
 (segment (start 103.8986 90.292) (end 103.136601 89.530001) (width 0.25) (layer F.Cu) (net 17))
 (segment (start 103.448009 92.649001) (end 104.420361 92.649001) (width 0.25) (layer F.Cu) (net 16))
 (segment (start 58.96 95.88) (end 56.46 93.38) (width 0.25) (layer F.Cu) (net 16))
 (segment (start 100.8506 95.88) (end 58.96 95.88) (width 0.25) (layer F.Cu) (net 16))
 (segment (start 103.8986 92.832) (end 100.8506 95.88) (width 0.25) (layer F.Cu) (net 16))
 (segment (start 118.356601 85.973999) (end 119.1186 85.212) (width 0.25) (layer F.Cu) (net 13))
 (segment (start 112.951599 91.379001) (end 118.356601 85.973999) (width 0.25) (layer F.Cu) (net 13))
 (segment (start 103.720999 91.379001) (end 112.951599 91.379001) (width 0.25) (layer F.Cu) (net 13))
 (segment (start 93.915999 94.415999) (end 100.784001 94.415999) (width 0.25) (layer F.Cu) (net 13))
 (segment (start 92.9 93.4) (end 93.915999 94.415999) (width 0.25) (layer F.Cu) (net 13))
 (segment (start 100.9 94.3) (end 103.720999 91.379001) (width 0.25) (layer F.Cu) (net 13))
 (segment (start 100.784001 94.415999) (end 100.9 94.3) (width 0.25) (layer F.Cu) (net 13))
 (segment (start 42.126009 89.813991) (end 100.227847 89.813991) (width 0.25) (layer B.Cu) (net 4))
 (segment (start 38.56 93.38) (end 42.126009 89.813991) (width 0.25) (layer B.Cu) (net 4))
 (segment (start 117.665601 89.204999) (end 118.356601 88.513999) (width 0.25) (layer B.Cu) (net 4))
 (segment (start 118.356601 88.513999) (end 119.1186 87.752) (width 0.25) (layer B.Cu) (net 4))
 (segment (start 100.836839 89.204999) (end 117.665601 89.204999) (width 0.25) (layer B.Cu) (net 4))
 (segment (start 100.227847 89.813991) (end 100.836839 89.204999) (width 0.25) (layer B.Cu) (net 4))
 (segment (start 103.136601 74.290001) (end 103.8986 75.052) (width 0.25) (layer F.Cu) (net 5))
 (segment (start 57.916319 72.938999) (end 101.785599 72.938999) (width 0.25) (layer F.Cu) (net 5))
 (segment (start 101.785599 72.938999) (end 103.136601 74.290001) (width 0.25) (layer F.Cu) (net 5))
 (segment (start 54.475318 76.38) (end 57.916319 72.938999) (width 0.25) (layer F.Cu) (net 5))
 (segment (start 38.56 76.38) (end 54.475318 76.38) (width 0.25) (layer F.Cu) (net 5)))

